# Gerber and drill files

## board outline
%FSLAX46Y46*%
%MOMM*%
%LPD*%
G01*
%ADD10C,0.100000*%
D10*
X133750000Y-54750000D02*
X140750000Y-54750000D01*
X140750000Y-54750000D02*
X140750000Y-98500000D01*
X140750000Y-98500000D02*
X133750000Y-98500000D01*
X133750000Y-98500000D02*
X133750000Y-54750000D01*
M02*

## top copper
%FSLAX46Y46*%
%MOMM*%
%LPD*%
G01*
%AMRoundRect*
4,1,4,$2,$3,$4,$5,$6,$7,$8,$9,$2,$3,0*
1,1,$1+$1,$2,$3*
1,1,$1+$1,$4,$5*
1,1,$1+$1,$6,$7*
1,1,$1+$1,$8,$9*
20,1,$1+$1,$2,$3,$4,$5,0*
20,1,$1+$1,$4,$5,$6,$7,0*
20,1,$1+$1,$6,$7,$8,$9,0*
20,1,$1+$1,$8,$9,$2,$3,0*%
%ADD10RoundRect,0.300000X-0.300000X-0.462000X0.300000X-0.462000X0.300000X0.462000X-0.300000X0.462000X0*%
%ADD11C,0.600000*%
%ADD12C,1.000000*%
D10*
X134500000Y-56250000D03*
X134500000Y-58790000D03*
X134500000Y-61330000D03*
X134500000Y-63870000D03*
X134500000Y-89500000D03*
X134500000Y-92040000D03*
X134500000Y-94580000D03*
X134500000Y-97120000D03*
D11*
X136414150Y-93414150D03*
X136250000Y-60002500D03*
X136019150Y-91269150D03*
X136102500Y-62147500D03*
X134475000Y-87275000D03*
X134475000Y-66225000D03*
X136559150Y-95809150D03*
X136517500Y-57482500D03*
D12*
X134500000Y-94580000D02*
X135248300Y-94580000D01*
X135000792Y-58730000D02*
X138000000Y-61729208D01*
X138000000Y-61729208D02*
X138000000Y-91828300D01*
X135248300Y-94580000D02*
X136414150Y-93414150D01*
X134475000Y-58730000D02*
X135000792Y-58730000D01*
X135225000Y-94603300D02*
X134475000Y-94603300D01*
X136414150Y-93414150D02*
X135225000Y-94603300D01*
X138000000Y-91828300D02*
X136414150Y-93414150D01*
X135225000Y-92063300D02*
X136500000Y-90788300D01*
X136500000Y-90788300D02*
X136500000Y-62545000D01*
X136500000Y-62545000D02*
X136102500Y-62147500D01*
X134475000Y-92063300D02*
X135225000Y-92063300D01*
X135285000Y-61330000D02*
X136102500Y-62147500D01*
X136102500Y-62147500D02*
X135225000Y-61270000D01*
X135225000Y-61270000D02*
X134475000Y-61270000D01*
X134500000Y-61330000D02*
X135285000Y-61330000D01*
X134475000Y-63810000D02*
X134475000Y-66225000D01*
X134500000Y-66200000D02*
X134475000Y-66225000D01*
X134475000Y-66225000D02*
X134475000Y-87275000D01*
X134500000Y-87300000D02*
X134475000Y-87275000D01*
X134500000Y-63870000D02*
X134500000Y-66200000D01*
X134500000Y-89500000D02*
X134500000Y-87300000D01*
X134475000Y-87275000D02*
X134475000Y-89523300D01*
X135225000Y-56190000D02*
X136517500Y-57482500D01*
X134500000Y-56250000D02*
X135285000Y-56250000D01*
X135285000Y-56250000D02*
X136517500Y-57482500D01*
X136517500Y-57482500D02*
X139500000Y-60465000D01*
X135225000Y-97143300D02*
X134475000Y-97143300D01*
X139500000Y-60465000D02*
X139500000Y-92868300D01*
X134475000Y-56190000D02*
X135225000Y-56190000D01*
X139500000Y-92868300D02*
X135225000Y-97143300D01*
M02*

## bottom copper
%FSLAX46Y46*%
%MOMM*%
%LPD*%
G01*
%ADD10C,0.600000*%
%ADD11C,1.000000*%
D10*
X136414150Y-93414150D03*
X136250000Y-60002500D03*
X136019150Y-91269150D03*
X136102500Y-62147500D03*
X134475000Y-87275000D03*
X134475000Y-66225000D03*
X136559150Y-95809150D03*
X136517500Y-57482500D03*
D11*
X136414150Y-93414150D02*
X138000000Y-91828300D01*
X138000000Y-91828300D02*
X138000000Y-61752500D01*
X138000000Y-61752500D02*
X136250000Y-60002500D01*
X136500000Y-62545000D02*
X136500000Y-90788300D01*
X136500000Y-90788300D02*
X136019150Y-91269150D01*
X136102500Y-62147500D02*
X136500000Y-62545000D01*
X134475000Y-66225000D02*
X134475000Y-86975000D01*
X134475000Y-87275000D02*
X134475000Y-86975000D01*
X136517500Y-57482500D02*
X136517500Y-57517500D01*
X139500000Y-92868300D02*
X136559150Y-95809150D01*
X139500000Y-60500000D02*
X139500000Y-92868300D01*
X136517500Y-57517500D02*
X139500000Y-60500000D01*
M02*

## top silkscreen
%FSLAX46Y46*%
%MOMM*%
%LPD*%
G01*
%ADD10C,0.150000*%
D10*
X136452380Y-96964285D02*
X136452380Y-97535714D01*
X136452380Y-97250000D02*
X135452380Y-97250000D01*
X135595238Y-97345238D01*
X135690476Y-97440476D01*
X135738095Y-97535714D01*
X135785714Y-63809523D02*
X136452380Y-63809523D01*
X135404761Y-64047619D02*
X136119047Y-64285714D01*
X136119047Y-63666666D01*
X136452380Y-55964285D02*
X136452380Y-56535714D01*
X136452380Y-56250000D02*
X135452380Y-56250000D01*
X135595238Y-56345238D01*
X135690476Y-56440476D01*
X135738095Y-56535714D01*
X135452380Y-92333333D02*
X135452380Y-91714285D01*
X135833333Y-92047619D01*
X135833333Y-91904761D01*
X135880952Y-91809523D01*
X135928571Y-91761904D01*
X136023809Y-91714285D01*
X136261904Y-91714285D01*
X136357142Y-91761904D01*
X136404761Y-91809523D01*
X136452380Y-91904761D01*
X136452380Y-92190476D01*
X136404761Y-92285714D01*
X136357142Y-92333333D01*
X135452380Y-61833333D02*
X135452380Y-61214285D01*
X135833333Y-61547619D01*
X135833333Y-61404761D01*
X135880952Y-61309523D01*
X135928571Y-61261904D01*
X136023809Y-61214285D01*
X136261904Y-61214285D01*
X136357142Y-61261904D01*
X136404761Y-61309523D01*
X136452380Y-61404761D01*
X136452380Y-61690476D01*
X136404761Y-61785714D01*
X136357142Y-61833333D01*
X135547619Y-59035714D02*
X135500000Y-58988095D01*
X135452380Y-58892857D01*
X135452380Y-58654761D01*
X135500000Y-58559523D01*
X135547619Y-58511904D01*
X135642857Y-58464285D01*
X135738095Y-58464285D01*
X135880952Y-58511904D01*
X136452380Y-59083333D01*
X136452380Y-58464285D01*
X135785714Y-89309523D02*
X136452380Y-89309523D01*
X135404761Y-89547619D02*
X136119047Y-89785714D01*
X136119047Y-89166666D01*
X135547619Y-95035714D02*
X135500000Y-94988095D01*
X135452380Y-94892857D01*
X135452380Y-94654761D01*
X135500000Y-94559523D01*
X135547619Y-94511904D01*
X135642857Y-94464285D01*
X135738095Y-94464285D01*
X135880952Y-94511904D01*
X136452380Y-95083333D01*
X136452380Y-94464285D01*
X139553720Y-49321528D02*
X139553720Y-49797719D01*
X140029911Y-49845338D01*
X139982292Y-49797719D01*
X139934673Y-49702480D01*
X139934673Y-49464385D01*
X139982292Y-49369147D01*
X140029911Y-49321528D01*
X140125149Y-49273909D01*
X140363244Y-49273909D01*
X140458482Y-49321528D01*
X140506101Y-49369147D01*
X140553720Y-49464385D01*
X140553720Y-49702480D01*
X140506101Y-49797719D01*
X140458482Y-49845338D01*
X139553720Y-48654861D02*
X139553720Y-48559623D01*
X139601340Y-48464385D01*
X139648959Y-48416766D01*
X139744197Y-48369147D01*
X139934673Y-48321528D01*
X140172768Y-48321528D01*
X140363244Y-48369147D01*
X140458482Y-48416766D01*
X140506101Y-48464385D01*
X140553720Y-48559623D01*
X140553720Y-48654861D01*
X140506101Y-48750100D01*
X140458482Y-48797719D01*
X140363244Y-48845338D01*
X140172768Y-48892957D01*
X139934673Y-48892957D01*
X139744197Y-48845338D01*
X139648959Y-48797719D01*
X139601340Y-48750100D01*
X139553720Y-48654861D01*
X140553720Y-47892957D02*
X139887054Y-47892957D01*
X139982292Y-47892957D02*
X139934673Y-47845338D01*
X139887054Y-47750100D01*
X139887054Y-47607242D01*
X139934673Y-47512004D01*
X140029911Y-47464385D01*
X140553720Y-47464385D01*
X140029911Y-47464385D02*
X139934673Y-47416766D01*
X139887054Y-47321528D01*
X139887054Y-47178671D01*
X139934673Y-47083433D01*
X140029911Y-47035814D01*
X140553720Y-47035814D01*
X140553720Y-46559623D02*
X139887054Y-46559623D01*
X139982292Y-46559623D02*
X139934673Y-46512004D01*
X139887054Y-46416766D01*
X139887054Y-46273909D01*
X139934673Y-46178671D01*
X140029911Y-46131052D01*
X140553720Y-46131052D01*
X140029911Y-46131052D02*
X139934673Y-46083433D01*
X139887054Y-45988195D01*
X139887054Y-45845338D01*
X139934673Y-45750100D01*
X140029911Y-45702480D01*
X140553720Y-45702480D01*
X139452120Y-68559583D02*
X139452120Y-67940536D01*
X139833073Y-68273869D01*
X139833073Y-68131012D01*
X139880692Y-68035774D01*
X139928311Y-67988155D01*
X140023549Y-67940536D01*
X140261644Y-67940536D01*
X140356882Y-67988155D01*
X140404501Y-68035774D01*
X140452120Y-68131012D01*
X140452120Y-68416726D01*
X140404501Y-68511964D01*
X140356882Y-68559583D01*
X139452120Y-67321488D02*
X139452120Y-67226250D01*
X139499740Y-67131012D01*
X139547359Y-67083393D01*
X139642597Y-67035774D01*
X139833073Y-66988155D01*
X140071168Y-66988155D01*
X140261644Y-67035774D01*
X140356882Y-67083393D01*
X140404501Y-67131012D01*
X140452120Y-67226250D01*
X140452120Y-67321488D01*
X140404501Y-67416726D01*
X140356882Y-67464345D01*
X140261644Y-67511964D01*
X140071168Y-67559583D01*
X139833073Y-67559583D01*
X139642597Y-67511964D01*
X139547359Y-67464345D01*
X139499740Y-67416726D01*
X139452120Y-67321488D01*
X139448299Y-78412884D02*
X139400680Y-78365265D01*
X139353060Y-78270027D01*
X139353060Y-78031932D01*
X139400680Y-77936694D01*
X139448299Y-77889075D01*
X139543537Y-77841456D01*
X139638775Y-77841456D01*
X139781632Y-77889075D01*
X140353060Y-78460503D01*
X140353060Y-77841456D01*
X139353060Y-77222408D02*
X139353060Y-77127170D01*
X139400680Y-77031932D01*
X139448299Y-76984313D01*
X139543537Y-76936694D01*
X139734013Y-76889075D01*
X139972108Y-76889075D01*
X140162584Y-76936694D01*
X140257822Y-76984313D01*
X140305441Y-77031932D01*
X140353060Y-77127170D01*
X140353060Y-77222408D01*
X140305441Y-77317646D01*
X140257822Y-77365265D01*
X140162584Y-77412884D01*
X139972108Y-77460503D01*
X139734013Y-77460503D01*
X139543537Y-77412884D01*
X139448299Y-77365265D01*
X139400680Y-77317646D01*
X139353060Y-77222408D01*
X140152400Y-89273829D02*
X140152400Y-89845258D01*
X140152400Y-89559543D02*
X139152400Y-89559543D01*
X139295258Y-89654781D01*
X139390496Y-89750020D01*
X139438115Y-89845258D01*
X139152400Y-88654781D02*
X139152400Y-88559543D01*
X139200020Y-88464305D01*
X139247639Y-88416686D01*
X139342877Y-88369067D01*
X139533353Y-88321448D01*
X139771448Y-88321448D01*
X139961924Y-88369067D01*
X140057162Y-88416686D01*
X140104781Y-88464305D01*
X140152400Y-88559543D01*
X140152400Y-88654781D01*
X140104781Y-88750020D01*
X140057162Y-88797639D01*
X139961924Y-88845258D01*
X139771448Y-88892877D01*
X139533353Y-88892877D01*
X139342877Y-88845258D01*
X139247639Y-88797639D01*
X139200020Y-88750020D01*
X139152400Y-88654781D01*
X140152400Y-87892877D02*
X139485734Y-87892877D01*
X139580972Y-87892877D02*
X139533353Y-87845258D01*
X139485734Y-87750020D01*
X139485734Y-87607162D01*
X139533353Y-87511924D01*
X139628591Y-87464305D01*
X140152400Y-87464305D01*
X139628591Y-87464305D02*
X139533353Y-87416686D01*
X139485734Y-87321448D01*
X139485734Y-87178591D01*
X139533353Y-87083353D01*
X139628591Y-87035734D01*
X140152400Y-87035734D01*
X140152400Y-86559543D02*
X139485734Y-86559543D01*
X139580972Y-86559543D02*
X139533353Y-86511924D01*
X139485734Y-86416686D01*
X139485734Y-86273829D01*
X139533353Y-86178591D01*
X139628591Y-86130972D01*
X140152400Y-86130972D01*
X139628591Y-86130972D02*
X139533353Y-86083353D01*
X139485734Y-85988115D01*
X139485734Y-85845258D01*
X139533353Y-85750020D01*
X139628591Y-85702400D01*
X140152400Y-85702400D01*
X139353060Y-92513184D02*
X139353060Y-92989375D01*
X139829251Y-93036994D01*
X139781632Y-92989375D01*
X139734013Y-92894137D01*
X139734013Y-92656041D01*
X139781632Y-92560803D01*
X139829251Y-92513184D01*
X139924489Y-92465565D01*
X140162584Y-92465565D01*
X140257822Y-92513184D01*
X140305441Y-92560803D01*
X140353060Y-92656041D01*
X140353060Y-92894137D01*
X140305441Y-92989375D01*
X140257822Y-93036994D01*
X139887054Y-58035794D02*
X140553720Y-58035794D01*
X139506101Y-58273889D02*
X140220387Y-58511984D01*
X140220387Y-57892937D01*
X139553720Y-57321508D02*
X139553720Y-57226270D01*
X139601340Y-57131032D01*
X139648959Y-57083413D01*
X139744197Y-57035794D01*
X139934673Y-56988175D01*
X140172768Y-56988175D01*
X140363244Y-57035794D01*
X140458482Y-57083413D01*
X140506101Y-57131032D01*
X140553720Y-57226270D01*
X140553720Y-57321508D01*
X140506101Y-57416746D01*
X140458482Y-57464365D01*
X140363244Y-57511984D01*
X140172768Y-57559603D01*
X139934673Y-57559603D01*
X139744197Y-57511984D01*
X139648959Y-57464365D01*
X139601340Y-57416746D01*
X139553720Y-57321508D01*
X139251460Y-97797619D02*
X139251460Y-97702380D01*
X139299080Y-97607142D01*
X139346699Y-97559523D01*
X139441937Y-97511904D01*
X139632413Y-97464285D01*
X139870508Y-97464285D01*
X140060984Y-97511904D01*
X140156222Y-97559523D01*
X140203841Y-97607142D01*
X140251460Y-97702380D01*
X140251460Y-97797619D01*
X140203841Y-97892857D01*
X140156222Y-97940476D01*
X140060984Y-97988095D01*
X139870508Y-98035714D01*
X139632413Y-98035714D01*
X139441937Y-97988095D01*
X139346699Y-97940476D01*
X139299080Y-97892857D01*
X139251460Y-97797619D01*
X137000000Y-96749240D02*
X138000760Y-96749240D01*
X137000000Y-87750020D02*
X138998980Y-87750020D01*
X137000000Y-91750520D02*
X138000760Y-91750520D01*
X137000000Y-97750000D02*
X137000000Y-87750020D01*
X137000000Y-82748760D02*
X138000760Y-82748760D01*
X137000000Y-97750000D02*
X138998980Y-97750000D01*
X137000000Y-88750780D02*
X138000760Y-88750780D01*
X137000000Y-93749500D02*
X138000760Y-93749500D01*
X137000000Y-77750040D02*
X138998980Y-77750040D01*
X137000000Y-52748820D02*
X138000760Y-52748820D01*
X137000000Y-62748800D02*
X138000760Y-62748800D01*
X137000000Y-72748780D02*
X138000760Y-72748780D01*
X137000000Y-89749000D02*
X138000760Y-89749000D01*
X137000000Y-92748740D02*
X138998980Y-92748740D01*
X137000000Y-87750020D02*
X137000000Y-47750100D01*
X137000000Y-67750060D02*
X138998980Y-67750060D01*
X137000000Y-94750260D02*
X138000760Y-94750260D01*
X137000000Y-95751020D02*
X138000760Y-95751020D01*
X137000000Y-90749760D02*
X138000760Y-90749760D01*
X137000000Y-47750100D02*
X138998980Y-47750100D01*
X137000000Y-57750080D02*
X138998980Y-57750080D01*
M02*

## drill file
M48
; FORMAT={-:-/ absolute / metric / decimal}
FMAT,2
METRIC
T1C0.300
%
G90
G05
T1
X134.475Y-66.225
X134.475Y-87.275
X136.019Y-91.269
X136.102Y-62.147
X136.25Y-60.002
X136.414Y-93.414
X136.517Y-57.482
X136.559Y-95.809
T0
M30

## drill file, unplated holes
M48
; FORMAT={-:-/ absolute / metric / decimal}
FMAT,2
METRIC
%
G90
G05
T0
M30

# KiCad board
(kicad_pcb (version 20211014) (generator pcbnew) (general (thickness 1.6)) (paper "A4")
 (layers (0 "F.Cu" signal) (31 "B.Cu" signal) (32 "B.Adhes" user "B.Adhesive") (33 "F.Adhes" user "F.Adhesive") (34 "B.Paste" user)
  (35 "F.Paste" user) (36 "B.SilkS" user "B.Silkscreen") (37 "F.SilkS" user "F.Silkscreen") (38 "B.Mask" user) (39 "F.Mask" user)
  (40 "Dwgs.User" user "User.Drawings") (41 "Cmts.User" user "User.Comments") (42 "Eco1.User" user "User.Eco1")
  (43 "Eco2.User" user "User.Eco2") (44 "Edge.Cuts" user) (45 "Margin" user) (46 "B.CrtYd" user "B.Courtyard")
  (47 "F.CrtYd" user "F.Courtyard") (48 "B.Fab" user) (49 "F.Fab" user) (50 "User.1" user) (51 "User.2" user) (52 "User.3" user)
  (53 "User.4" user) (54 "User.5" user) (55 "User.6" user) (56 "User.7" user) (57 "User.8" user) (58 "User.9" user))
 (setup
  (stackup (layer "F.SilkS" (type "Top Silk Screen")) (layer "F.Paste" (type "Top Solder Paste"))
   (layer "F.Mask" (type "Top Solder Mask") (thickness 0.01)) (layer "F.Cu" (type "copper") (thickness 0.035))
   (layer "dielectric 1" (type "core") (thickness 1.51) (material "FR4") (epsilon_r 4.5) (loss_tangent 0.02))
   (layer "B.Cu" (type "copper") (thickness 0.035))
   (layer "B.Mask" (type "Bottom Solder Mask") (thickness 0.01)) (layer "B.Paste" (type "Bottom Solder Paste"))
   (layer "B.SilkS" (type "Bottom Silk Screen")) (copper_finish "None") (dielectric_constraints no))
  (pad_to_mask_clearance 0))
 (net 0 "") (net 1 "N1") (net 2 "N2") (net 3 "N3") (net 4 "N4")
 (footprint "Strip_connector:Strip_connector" (layer "F.Cu") (at 134.5 56.25)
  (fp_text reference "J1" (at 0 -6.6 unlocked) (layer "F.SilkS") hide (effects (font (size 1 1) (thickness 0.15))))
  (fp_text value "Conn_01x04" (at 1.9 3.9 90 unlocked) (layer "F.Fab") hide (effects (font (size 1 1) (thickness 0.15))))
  (pad "1" smd roundrect (at 0 0) (size 1.2 1.524) (layers "F.Cu" "F.Paste" "F.Mask") (roundrect_rratio 0.25) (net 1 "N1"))
  (pad "2" smd roundrect (at 0 2.54) (size 1.2 1.524) (layers "F.Cu" "F.Paste" "F.Mask") (roundrect_rratio 0.25) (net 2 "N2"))
  (pad "3" smd roundrect (at 0 5.08) (size 1.2 1.524) (layers "F.Cu" "F.Paste" "F.Mask") (roundrect_rratio 0.25) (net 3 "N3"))
  (pad "4" smd roundrect (at 0 7.62) (size 1.2 1.524) (layers "F.Cu" "F.Paste" "F.Mask") (roundrect_rratio 0.25) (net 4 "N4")))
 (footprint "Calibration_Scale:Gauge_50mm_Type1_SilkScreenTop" (layer "F.Cu") (at 137 97.75 90)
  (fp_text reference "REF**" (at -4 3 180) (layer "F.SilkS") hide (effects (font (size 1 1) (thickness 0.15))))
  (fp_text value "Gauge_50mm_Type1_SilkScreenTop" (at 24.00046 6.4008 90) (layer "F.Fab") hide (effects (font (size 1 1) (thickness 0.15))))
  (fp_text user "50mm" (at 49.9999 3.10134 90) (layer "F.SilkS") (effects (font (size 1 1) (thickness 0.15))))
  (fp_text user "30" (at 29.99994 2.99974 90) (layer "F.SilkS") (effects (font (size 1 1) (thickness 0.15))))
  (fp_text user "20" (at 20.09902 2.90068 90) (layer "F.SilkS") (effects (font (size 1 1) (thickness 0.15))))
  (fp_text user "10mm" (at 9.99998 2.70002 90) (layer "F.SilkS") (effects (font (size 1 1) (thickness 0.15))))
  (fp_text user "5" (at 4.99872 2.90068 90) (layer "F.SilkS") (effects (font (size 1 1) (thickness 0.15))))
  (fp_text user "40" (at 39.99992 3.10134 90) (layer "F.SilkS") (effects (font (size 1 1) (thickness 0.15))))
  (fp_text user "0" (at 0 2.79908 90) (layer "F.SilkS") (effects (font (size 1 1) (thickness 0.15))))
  (fp_line (start 1.00076 0) (end 1.00076 1.00076) (layer "F.SilkS") (width 0.15))
  (fp_line (start 9.99998 0) (end 9.99998 1.99898) (layer "F.SilkS") (width 0.15))
  (fp_line (start 5.99948 0) (end 5.99948 1.00076) (layer "F.SilkS") (width 0.15))
  (fp_line (start 0 0) (end 9.99998 0) (layer "F.SilkS") (width 0.15))
  (fp_line (start 15.00124 0) (end 15.00124 1.00076) (layer "F.SilkS") (width 0.15))
  (fp_line (start 0 0) (end 0 1.99898) (layer "F.SilkS") (width 0.15))
  (fp_line (start 8.99922 0) (end 8.99922 1.00076) (layer "F.SilkS") (width 0.15))
  (fp_line (start 4.0005 0) (end 4.0005 1.00076) (layer "F.SilkS") (width 0.15))
  (fp_line (start 19.99996 0) (end 19.99996 1.99898) (layer "F.SilkS") (width 0.15))
  (fp_line (start 45.00118 0) (end 45.00118 1.00076) (layer "F.SilkS") (width 0.15))
  (fp_line (start 35.0012 0) (end 35.0012 1.00076) (layer "F.SilkS") (width 0.15))
  (fp_line (start 25.00122 0) (end 25.00122 1.00076) (layer "F.SilkS") (width 0.15))
  (fp_line (start 8.001 0) (end 8.001 1.00076) (layer "F.SilkS") (width 0.15))
  (fp_line (start 5.00126 0) (end 5.00126 1.99898) (layer "F.SilkS") (width 0.15))
  (fp_line (start 9.99998 0) (end 49.9999 0) (layer "F.SilkS") (width 0.15))
  (fp_line (start 29.99994 0) (end 29.99994 1.99898) (layer "F.SilkS") (width 0.15))
  (fp_line (start 2.99974 0) (end 2.99974 1.00076) (layer "F.SilkS") (width 0.15))
  (fp_line (start 1.99898 0) (end 1.99898 1.00076) (layer "F.SilkS") (width 0.15))
  (fp_line (start 7.00024 0) (end 7.00024 1.00076) (layer "F.SilkS") (width 0.15))
  (fp_line (start 49.9999 0) (end 49.9999 1.99898) (layer "F.SilkS") (width 0.15))
  (fp_line (start 39.99992 0) (end 39.99992 1.99898) (layer "F.SilkS") (width 0.15)))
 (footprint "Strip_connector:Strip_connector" (layer "F.Cu") (at 134.5 89.5)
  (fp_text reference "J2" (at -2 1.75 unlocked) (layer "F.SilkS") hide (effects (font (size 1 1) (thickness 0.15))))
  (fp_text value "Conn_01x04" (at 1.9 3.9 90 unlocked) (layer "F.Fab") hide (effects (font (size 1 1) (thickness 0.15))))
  (pad "1" smd roundrect (at 0 0) (size 1.2 1.524) (layers "F.Cu" "F.Paste" "F.Mask") (roundrect_rratio 0.25) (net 4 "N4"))
  (pad "2" smd roundrect (at 0 2.54) (size 1.2 1.524) (layers "F.Cu" "F.Paste" "F.Mask") (roundrect_rratio 0.25) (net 3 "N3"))
  (pad "3" smd roundrect (at 0 5.08) (size 1.2 1.524) (layers "F.Cu" "F.Paste" "F.Mask") (roundrect_rratio 0.25) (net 2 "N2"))
  (pad "4" smd roundrect (at 0 7.62) (size 1.2 1.524) (layers "F.Cu" "F.Paste" "F.Mask") (roundrect_rratio 0.25) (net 1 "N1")))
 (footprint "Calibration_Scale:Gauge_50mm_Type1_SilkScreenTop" (layer "B.Cu") (at 133.75 54.75 -90)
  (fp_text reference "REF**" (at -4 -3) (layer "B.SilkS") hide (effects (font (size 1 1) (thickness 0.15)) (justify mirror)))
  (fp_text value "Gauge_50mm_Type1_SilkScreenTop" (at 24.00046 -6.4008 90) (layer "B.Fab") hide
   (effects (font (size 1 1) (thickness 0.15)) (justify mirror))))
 (gr_rect (start 133.75 54.75) (end 140.75 98.5) (layer "Edge.Cuts") (width 0.1) (fill none))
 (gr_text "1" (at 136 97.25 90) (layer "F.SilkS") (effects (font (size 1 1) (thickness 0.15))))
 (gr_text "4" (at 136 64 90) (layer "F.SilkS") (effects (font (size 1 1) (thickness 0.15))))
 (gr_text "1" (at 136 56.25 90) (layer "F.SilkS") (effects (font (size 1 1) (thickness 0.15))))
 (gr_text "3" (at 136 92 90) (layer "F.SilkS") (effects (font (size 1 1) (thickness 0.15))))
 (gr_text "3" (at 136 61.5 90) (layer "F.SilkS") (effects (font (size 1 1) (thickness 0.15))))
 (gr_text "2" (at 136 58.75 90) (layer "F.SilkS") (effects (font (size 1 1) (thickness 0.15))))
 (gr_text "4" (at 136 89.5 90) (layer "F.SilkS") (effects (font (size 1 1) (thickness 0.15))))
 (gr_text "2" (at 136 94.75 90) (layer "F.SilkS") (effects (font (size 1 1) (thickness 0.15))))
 (segment (start 134.5 94.58) (end 135.2483 94.58) (width 1) (layer "F.Cu") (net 2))
 (segment (start 135.000792 58.73) (end 138 61.729208) (width 1) (layer "F.Cu") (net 2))
 (segment (start 138 61.729208) (end 138 91.8283) (width 1) (layer "F.Cu") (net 2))
 (segment (start 135.2483 94.58) (end 136.41415 93.41415) (width 1) (layer "F.Cu") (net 2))
 (segment (start 134.475 58.73) (end 135.000792 58.73) (width 1) (layer "F.Cu") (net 2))
 (segment (start 135.225 94.6033) (end 134.475 94.6033) (width 1) (layer "F.Cu") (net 2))
 (segment (start 136.41415 93.41415) (end 135.225 94.6033) (width 1) (layer "F.Cu") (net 2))
 (segment (start 138 91.8283) (end 136.41415 93.41415) (width 1) (layer "F.Cu") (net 2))
 (via (at 136.41415 93.41415) (size 0.6) (drill 0.3) (layers "F.Cu" "B.Cu") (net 2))
 (via (at 136.25 60.0025) (size 0.6) (drill 0.3) (layers "F.Cu" "B.Cu") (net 2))
 (segment (start 136.41415 93.41415) (end 138 91.8283) (width 1) (layer "B.Cu") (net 2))
 (segment (start 138 91.8283) (end 138 61.7525) (width 1) (layer "B.Cu") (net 2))
 (segment (start 138 61.7525) (end 136.25 60.0025) (width 1) (layer "B.Cu") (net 2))
 (segment (start 135.225 92.0633) (end 136.5 90.7883) (width 1) (layer "F.Cu") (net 3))
 (segment (start 136.5 90.7883) (end 136.5 62.545) (width 1) (layer "F.Cu") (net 3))
 (segment (start 136.5 62.545) (end 136.1025 62.1475) (width 1) (layer "F.Cu") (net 3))
 (segment (start 134.475 92.0633) (end 135.225 92.0633) (width 1) (layer "F.Cu") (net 3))
 (segment (start 135.285 61.33) (end 136.1025 62.1475) (width 1) (layer "F.Cu") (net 3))
 (segment (start 136.1025 62.1475) (end 135.225 61.27) (width 1) (layer "F.Cu") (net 3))
 (segment (start 135.225 61.27) (end 134.475 61.27) (width 1) (layer "F.Cu") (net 3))
 (segment (start 134.5 61.33) (end 135.285 61.33) (width 1) (layer "F.Cu") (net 3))
 (via (at 136.01915 91.26915) (size 0.6) (drill 0.3) (layers "F.Cu" "B.Cu") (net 3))
 (via (at 136.1025 62.1475) (size 0.6) (drill 0.3) (layers "F.Cu" "B.Cu") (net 3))
 (segment (start 136.5 62.545) (end 136.5 90.7883) (width 1) (layer "B.Cu") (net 3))
 (segment (start 136.5 90.7883) (end 136.01915 91.26915) (width 1) (layer "B.Cu") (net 3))
 (segment (start 136.1025 62.1475) (end 136.5 62.545) (width 1) (layer "B.Cu") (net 3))
 (segment (start 134.475 63.81) (end 134.475 66.225) (width 1) (layer "F.Cu") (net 4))
 (segment (start 134.5 66.2) (end 134.475 66.225) (width 1) (layer "F.Cu") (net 4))
 (segment (start 134.475 66.225) (end 134.475 87.275) (width 1) (layer "F.Cu") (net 4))
 (segment (start 134.5 87.3) (end 134.475 87.275) (width 1) (layer "F.Cu") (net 4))
 (segment (start 134.5 63.87) (end 134.5 66.2) (width 1) (layer "F.Cu") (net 4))
 (segment (start 134.5 89.5) (end 134.5 87.3) (width 1) (layer "F.Cu") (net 4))
 (segment (start 134.475 87.275) (end 134.475 89.5233) (width 1) (layer "F.Cu") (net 4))
 (via (at 134.475 87.275) (size 0.6) (drill 0.3) (layers "F.Cu" "B.Cu") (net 4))
 (via (at 134.475 66.225) (size 0.6) (drill 0.3) (layers "F.Cu" "B.Cu") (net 4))
 (segment (start 134.475 66.225) (end 134.475 86.975) (width 1) (layer "B.Cu") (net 4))
 (segment (start 134.475 87.275) (end 134.475 86.975) (width 1) (layer "B.Cu") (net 4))
 (segment (start 135.225 56.19) (end 136.5175 57.4825) (width 1) (layer "F.Cu") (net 1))
 (segment (start 134.5 56.25) (end 135.285 56.25) (width 1) (layer "F.Cu") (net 1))
 (segment (start 135.285 56.25) (end 136.5175 57.4825) (width 1) (layer "F.Cu") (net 1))
 (segment (start 136.5175 57.4825) (end 139.5 60.465) (width 1) (layer "F.Cu") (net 1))
 (segment (start 135.225 97.1433) (end 134.475 97.1433) (width 1) (layer "F.Cu") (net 1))
 (segment (start 139.5 60.465) (end 139.5 92.8683) (width 1) (layer "F.Cu") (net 1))
 (segment (start 134.475 56.19) (end 135.225 56.19) (width 1) (layer "F.Cu") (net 1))
 (segment (start 139.5 92.8683) (end 135.225 97.1433) (width 1) (layer "F.Cu") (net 1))
 (via (at 136.55915 95.80915) (size 0.6) (drill 0.3) (layers "F.Cu" "B.Cu") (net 1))
 (via (at 136.5175 57.4825) (size 0.6) (drill 0.3) (layers "F.Cu" "B.Cu") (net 1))
 (segment (start 136.5175 57.4825) (end 136.5175 57.5175) (width 1) (layer "B.Cu") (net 1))
 (segment (start 139.5 92.8683) (end 136.55915 95.80915) (width 1) (layer "B.Cu") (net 1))
 (segment (start 139.5 60.5) (end 139.5 92.8683) (width 1) (layer "B.Cu") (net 1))
 (segment (start 136.5175 57.5175) (end 139.5 60.5) (width 1) (layer "B.Cu") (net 1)))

